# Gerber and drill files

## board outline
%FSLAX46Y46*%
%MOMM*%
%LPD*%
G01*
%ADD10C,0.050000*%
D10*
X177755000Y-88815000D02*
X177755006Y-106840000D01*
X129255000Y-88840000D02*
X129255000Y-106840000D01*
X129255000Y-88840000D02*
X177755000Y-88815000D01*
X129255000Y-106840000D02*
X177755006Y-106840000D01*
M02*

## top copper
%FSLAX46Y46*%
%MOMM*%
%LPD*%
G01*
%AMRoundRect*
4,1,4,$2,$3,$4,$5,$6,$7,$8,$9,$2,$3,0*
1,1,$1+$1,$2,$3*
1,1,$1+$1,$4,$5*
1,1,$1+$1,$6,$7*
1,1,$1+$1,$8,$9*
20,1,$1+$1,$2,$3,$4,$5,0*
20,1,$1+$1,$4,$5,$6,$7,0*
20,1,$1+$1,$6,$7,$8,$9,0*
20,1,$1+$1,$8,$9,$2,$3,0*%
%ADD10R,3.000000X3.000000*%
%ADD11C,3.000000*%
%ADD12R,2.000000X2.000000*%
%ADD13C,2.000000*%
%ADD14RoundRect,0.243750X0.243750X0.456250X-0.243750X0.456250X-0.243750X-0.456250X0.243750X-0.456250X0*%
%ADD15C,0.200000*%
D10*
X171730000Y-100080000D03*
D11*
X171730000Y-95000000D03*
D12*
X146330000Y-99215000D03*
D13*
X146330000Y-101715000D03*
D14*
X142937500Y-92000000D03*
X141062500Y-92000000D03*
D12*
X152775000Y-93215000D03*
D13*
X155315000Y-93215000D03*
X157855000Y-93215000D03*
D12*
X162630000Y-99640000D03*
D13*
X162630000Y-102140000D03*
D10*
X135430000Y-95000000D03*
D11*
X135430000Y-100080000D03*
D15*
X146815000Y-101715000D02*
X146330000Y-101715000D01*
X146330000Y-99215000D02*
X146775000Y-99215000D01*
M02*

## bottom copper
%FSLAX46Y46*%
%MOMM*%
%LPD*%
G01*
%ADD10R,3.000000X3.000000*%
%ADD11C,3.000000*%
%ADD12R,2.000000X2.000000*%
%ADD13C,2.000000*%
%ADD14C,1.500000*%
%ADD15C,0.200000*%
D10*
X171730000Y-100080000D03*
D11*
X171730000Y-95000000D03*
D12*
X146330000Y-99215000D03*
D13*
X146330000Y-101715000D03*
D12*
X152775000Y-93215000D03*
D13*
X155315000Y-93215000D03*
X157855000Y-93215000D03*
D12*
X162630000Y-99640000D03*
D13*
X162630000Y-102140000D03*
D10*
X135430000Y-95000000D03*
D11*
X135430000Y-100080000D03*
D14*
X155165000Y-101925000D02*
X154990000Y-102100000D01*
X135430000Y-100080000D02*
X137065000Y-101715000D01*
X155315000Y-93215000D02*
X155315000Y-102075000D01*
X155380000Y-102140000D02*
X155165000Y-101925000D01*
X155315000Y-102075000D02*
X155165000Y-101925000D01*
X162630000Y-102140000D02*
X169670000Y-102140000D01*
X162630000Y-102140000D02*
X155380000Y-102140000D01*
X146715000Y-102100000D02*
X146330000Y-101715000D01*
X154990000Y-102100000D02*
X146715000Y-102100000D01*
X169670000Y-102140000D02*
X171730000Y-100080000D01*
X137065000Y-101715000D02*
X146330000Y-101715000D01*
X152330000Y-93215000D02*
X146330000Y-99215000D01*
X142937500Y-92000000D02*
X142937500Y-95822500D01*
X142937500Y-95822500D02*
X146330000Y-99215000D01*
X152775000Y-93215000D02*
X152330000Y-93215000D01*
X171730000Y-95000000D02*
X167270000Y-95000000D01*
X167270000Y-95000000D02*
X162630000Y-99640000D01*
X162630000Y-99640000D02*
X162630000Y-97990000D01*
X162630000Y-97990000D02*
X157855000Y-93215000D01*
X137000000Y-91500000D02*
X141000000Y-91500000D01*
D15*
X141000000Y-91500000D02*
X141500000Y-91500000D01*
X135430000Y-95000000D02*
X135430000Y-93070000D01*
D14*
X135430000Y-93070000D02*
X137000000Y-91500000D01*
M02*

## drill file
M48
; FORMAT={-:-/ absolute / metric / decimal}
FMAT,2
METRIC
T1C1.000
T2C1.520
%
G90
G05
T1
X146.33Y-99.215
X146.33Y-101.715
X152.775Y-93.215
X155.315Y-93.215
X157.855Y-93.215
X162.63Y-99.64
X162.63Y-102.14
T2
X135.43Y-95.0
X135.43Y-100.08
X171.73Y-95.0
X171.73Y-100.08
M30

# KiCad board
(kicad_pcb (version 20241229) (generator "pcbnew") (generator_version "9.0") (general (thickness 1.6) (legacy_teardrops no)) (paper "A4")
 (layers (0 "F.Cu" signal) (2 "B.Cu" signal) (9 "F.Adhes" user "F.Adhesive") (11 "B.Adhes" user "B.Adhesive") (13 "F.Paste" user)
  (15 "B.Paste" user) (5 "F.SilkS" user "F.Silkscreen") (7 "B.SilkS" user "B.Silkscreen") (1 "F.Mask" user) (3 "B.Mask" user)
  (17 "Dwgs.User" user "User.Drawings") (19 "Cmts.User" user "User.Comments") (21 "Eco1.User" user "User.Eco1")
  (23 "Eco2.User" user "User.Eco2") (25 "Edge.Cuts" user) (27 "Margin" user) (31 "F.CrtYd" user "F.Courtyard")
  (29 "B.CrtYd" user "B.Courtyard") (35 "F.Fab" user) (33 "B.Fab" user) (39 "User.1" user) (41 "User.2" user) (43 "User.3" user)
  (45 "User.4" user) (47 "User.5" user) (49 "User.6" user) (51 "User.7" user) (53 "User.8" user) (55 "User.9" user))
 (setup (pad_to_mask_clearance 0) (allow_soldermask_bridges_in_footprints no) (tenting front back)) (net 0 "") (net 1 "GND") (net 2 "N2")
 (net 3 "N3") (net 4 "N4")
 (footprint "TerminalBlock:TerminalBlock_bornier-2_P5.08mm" (layer "F.Cu") (at 171.73 100.08 90)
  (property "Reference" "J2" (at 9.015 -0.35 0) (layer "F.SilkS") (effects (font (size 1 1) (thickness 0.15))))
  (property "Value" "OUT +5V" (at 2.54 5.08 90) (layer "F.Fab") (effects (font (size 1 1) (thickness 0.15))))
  (pad "1" thru_hole rect (at 0 0 90) (size 3 3) (drill 1.52) (layers "*.Cu" "*.Mask") (remove_unused_layers no) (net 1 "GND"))
  (pad "2" thru_hole circle (at 5.08 0 90) (size 3 3) (drill 1.52) (layers "*.Cu" "*.Mask") (remove_unused_layers no) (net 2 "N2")))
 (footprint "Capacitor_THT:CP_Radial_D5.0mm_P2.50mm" (layer "F.Cu") (at 146.33 99.215 -90)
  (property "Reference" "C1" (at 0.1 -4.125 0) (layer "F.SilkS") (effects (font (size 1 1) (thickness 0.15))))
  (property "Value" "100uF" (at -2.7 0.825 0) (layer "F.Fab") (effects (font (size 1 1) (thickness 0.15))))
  (pad "1" thru_hole rect (at 0 0 270) (size 2 2) (drill 1) (layers "*.Cu" "*.Mask") (remove_unused_layers no) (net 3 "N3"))
  (pad "2" thru_hole circle (at 2.5 0 270) (size 2 2) (drill 1) (layers "*.Cu" "*.Mask") (remove_unused_layers no) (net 1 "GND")))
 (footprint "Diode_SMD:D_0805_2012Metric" (layer "F.Cu") (at 142 92 180)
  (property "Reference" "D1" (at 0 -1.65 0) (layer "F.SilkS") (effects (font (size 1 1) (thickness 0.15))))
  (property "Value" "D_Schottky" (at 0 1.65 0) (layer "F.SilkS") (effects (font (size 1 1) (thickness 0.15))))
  (pad "1" smd roundrect (at -0.9375 0 180) (size 0.975 1.4) (layers "F.Cu" "F.Mask" "F.Paste") (roundrect_rratio 0.25) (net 3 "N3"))
  (pad "2" smd roundrect (at 0.9375 0 180) (size 0.975 1.4) (layers "F.Cu" "F.Mask" "F.Paste") (roundrect_rratio 0.25) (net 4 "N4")))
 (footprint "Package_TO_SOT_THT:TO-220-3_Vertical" (layer "F.Cu") (at 152.775 93.215)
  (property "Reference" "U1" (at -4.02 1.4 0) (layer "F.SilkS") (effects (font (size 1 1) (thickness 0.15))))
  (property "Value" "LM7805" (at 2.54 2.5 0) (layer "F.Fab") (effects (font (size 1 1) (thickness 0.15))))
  (pad "1" thru_hole rect (at 0 0) (size 2 2) (drill 1) (layers "*.Cu" "*.Mask") (remove_unused_layers no) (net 3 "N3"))
  (pad "2" thru_hole circle (at 2.54 0) (size 2 2) (drill 1) (layers "*.Cu" "*.Mask") (remove_unused_layers no) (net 1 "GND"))
  (pad "3" thru_hole circle (at 5.08 0) (size 2 2) (drill 1) (layers "*.Cu" "*.Mask") (remove_unused_layers no) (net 2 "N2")))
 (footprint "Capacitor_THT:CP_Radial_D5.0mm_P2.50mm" (layer "F.Cu") (at 162.63 99.64 -90)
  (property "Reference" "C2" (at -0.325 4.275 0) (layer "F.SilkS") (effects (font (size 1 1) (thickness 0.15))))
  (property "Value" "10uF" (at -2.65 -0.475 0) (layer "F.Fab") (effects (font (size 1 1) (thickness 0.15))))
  (pad "1" thru_hole rect (at 0 0 270) (size 2 2) (drill 1) (layers "*.Cu" "*.Mask") (remove_unused_layers no) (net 2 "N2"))
  (pad "2" thru_hole circle (at 2.5 0 270) (size 2 2) (drill 1) (layers "*.Cu" "*.Mask") (remove_unused_layers no) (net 1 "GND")))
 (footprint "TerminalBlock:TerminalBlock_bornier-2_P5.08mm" (layer "F.Cu") (at 135.43 95 -90)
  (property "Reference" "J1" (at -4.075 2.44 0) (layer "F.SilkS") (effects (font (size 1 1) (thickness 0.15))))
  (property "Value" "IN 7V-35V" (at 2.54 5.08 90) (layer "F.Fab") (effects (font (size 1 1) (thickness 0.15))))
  (pad "1" thru_hole rect (at 0 0 270) (size 3 3) (drill 1.52) (layers "*.Cu" "*.Mask") (remove_unused_layers no) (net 4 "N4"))
  (pad "2" thru_hole circle (at 5.08 0 270) (size 3 3) (drill 1.52) (layers "*.Cu" "*.Mask") (remove_unused_layers no) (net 1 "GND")))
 (gr_line (start 177.755 88.815) (end 177.755006 106.84) (stroke (width 0.05) (type default)) (layer "Edge.Cuts"))
 (gr_line (start 129.255 88.84) (end 129.255 106.84) (stroke (width 0.05) (type default)) (layer "Edge.Cuts"))
 (gr_line (start 129.255 88.84) (end 177.755 88.815) (stroke (width 0.05) (type default)) (layer "Edge.Cuts"))
 (gr_line (start 129.255 106.84) (end 177.755006 106.84) (stroke (width 0.05) (type default)) (layer "Edge.Cuts"))
 (segment (start 146.815 101.715) (end 146.33 101.715) (width 0.2) (layer "F.Cu") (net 1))
 (segment (start 155.165 101.925) (end 154.99 102.1) (width 1.5) (layer "B.Cu") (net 1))
 (segment (start 135.43 100.08) (end 137.065 101.715) (width 1.5) (layer "B.Cu") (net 1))
 (segment (start 155.315 93.215) (end 155.315 102.075) (width 1.5) (layer "B.Cu") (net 1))
 (segment (start 155.38 102.14) (end 155.165 101.925) (width 1.5) (layer "B.Cu") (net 1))
 (segment (start 155.315 102.075) (end 155.165 101.925) (width 1.5) (layer "B.Cu") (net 1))
 (segment (start 162.63 102.14) (end 169.67 102.14) (width 1.5) (layer "B.Cu") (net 1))
 (segment (start 162.63 102.14) (end 155.38 102.14) (width 1.5) (layer "B.Cu") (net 1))
 (segment (start 146.715 102.1) (end 146.33 101.715) (width 1.5) (layer "B.Cu") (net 1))
 (segment (start 154.99 102.1) (end 146.715 102.1) (width 1.5) (layer "B.Cu") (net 1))
 (segment (start 169.67 102.14) (end 171.73 100.08) (width 1.5) (layer "B.Cu") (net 1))
 (segment (start 137.065 101.715) (end 146.33 101.715) (width 1.5) (layer "B.Cu") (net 1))
 (segment (start 146.33 99.215) (end 146.775 99.215) (width 0.2) (layer "F.Cu") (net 3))
 (segment (start 152.33 93.215) (end 146.33 99.215) (width 1.5) (layer "B.Cu") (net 3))
 (segment (start 142.9375 92) (end 142.9375 95.8225) (width 1.5) (layer "B.Cu") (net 3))
 (segment (start 142.9375 95.8225) (end 146.33 99.215) (width 1.5) (layer "B.Cu") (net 3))
 (segment (start 152.775 93.215) (end 152.33 93.215) (width 1.5) (layer "B.Cu") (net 3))
 (segment (start 171.73 95) (end 167.27 95) (width 1.5) (layer "B.Cu") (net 2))
 (segment (start 167.27 95) (end 162.63 99.64) (width 1.5) (layer "B.Cu") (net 2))
 (segment (start 162.63 99.64) (end 162.63 97.99) (width 1.5) (layer "B.Cu") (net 2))
 (segment (start 162.63 97.99) (end 157.855 93.215) (width 1.5) (layer "B.Cu") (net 2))
 (segment (start 137 91.5) (end 141 91.5) (width 1.5) (layer "B.Cu") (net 4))
 (segment (start 141 91.5) (end 141.5 91.5) (width 0.2) (layer "B.Cu") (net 4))
 (segment (start 135.43 95) (end 135.43 93.07) (width 0.2) (layer "B.Cu") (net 4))
 (segment (start 135.43 93.07) (end 137 91.5) (width 1.5) (layer "B.Cu") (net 4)))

